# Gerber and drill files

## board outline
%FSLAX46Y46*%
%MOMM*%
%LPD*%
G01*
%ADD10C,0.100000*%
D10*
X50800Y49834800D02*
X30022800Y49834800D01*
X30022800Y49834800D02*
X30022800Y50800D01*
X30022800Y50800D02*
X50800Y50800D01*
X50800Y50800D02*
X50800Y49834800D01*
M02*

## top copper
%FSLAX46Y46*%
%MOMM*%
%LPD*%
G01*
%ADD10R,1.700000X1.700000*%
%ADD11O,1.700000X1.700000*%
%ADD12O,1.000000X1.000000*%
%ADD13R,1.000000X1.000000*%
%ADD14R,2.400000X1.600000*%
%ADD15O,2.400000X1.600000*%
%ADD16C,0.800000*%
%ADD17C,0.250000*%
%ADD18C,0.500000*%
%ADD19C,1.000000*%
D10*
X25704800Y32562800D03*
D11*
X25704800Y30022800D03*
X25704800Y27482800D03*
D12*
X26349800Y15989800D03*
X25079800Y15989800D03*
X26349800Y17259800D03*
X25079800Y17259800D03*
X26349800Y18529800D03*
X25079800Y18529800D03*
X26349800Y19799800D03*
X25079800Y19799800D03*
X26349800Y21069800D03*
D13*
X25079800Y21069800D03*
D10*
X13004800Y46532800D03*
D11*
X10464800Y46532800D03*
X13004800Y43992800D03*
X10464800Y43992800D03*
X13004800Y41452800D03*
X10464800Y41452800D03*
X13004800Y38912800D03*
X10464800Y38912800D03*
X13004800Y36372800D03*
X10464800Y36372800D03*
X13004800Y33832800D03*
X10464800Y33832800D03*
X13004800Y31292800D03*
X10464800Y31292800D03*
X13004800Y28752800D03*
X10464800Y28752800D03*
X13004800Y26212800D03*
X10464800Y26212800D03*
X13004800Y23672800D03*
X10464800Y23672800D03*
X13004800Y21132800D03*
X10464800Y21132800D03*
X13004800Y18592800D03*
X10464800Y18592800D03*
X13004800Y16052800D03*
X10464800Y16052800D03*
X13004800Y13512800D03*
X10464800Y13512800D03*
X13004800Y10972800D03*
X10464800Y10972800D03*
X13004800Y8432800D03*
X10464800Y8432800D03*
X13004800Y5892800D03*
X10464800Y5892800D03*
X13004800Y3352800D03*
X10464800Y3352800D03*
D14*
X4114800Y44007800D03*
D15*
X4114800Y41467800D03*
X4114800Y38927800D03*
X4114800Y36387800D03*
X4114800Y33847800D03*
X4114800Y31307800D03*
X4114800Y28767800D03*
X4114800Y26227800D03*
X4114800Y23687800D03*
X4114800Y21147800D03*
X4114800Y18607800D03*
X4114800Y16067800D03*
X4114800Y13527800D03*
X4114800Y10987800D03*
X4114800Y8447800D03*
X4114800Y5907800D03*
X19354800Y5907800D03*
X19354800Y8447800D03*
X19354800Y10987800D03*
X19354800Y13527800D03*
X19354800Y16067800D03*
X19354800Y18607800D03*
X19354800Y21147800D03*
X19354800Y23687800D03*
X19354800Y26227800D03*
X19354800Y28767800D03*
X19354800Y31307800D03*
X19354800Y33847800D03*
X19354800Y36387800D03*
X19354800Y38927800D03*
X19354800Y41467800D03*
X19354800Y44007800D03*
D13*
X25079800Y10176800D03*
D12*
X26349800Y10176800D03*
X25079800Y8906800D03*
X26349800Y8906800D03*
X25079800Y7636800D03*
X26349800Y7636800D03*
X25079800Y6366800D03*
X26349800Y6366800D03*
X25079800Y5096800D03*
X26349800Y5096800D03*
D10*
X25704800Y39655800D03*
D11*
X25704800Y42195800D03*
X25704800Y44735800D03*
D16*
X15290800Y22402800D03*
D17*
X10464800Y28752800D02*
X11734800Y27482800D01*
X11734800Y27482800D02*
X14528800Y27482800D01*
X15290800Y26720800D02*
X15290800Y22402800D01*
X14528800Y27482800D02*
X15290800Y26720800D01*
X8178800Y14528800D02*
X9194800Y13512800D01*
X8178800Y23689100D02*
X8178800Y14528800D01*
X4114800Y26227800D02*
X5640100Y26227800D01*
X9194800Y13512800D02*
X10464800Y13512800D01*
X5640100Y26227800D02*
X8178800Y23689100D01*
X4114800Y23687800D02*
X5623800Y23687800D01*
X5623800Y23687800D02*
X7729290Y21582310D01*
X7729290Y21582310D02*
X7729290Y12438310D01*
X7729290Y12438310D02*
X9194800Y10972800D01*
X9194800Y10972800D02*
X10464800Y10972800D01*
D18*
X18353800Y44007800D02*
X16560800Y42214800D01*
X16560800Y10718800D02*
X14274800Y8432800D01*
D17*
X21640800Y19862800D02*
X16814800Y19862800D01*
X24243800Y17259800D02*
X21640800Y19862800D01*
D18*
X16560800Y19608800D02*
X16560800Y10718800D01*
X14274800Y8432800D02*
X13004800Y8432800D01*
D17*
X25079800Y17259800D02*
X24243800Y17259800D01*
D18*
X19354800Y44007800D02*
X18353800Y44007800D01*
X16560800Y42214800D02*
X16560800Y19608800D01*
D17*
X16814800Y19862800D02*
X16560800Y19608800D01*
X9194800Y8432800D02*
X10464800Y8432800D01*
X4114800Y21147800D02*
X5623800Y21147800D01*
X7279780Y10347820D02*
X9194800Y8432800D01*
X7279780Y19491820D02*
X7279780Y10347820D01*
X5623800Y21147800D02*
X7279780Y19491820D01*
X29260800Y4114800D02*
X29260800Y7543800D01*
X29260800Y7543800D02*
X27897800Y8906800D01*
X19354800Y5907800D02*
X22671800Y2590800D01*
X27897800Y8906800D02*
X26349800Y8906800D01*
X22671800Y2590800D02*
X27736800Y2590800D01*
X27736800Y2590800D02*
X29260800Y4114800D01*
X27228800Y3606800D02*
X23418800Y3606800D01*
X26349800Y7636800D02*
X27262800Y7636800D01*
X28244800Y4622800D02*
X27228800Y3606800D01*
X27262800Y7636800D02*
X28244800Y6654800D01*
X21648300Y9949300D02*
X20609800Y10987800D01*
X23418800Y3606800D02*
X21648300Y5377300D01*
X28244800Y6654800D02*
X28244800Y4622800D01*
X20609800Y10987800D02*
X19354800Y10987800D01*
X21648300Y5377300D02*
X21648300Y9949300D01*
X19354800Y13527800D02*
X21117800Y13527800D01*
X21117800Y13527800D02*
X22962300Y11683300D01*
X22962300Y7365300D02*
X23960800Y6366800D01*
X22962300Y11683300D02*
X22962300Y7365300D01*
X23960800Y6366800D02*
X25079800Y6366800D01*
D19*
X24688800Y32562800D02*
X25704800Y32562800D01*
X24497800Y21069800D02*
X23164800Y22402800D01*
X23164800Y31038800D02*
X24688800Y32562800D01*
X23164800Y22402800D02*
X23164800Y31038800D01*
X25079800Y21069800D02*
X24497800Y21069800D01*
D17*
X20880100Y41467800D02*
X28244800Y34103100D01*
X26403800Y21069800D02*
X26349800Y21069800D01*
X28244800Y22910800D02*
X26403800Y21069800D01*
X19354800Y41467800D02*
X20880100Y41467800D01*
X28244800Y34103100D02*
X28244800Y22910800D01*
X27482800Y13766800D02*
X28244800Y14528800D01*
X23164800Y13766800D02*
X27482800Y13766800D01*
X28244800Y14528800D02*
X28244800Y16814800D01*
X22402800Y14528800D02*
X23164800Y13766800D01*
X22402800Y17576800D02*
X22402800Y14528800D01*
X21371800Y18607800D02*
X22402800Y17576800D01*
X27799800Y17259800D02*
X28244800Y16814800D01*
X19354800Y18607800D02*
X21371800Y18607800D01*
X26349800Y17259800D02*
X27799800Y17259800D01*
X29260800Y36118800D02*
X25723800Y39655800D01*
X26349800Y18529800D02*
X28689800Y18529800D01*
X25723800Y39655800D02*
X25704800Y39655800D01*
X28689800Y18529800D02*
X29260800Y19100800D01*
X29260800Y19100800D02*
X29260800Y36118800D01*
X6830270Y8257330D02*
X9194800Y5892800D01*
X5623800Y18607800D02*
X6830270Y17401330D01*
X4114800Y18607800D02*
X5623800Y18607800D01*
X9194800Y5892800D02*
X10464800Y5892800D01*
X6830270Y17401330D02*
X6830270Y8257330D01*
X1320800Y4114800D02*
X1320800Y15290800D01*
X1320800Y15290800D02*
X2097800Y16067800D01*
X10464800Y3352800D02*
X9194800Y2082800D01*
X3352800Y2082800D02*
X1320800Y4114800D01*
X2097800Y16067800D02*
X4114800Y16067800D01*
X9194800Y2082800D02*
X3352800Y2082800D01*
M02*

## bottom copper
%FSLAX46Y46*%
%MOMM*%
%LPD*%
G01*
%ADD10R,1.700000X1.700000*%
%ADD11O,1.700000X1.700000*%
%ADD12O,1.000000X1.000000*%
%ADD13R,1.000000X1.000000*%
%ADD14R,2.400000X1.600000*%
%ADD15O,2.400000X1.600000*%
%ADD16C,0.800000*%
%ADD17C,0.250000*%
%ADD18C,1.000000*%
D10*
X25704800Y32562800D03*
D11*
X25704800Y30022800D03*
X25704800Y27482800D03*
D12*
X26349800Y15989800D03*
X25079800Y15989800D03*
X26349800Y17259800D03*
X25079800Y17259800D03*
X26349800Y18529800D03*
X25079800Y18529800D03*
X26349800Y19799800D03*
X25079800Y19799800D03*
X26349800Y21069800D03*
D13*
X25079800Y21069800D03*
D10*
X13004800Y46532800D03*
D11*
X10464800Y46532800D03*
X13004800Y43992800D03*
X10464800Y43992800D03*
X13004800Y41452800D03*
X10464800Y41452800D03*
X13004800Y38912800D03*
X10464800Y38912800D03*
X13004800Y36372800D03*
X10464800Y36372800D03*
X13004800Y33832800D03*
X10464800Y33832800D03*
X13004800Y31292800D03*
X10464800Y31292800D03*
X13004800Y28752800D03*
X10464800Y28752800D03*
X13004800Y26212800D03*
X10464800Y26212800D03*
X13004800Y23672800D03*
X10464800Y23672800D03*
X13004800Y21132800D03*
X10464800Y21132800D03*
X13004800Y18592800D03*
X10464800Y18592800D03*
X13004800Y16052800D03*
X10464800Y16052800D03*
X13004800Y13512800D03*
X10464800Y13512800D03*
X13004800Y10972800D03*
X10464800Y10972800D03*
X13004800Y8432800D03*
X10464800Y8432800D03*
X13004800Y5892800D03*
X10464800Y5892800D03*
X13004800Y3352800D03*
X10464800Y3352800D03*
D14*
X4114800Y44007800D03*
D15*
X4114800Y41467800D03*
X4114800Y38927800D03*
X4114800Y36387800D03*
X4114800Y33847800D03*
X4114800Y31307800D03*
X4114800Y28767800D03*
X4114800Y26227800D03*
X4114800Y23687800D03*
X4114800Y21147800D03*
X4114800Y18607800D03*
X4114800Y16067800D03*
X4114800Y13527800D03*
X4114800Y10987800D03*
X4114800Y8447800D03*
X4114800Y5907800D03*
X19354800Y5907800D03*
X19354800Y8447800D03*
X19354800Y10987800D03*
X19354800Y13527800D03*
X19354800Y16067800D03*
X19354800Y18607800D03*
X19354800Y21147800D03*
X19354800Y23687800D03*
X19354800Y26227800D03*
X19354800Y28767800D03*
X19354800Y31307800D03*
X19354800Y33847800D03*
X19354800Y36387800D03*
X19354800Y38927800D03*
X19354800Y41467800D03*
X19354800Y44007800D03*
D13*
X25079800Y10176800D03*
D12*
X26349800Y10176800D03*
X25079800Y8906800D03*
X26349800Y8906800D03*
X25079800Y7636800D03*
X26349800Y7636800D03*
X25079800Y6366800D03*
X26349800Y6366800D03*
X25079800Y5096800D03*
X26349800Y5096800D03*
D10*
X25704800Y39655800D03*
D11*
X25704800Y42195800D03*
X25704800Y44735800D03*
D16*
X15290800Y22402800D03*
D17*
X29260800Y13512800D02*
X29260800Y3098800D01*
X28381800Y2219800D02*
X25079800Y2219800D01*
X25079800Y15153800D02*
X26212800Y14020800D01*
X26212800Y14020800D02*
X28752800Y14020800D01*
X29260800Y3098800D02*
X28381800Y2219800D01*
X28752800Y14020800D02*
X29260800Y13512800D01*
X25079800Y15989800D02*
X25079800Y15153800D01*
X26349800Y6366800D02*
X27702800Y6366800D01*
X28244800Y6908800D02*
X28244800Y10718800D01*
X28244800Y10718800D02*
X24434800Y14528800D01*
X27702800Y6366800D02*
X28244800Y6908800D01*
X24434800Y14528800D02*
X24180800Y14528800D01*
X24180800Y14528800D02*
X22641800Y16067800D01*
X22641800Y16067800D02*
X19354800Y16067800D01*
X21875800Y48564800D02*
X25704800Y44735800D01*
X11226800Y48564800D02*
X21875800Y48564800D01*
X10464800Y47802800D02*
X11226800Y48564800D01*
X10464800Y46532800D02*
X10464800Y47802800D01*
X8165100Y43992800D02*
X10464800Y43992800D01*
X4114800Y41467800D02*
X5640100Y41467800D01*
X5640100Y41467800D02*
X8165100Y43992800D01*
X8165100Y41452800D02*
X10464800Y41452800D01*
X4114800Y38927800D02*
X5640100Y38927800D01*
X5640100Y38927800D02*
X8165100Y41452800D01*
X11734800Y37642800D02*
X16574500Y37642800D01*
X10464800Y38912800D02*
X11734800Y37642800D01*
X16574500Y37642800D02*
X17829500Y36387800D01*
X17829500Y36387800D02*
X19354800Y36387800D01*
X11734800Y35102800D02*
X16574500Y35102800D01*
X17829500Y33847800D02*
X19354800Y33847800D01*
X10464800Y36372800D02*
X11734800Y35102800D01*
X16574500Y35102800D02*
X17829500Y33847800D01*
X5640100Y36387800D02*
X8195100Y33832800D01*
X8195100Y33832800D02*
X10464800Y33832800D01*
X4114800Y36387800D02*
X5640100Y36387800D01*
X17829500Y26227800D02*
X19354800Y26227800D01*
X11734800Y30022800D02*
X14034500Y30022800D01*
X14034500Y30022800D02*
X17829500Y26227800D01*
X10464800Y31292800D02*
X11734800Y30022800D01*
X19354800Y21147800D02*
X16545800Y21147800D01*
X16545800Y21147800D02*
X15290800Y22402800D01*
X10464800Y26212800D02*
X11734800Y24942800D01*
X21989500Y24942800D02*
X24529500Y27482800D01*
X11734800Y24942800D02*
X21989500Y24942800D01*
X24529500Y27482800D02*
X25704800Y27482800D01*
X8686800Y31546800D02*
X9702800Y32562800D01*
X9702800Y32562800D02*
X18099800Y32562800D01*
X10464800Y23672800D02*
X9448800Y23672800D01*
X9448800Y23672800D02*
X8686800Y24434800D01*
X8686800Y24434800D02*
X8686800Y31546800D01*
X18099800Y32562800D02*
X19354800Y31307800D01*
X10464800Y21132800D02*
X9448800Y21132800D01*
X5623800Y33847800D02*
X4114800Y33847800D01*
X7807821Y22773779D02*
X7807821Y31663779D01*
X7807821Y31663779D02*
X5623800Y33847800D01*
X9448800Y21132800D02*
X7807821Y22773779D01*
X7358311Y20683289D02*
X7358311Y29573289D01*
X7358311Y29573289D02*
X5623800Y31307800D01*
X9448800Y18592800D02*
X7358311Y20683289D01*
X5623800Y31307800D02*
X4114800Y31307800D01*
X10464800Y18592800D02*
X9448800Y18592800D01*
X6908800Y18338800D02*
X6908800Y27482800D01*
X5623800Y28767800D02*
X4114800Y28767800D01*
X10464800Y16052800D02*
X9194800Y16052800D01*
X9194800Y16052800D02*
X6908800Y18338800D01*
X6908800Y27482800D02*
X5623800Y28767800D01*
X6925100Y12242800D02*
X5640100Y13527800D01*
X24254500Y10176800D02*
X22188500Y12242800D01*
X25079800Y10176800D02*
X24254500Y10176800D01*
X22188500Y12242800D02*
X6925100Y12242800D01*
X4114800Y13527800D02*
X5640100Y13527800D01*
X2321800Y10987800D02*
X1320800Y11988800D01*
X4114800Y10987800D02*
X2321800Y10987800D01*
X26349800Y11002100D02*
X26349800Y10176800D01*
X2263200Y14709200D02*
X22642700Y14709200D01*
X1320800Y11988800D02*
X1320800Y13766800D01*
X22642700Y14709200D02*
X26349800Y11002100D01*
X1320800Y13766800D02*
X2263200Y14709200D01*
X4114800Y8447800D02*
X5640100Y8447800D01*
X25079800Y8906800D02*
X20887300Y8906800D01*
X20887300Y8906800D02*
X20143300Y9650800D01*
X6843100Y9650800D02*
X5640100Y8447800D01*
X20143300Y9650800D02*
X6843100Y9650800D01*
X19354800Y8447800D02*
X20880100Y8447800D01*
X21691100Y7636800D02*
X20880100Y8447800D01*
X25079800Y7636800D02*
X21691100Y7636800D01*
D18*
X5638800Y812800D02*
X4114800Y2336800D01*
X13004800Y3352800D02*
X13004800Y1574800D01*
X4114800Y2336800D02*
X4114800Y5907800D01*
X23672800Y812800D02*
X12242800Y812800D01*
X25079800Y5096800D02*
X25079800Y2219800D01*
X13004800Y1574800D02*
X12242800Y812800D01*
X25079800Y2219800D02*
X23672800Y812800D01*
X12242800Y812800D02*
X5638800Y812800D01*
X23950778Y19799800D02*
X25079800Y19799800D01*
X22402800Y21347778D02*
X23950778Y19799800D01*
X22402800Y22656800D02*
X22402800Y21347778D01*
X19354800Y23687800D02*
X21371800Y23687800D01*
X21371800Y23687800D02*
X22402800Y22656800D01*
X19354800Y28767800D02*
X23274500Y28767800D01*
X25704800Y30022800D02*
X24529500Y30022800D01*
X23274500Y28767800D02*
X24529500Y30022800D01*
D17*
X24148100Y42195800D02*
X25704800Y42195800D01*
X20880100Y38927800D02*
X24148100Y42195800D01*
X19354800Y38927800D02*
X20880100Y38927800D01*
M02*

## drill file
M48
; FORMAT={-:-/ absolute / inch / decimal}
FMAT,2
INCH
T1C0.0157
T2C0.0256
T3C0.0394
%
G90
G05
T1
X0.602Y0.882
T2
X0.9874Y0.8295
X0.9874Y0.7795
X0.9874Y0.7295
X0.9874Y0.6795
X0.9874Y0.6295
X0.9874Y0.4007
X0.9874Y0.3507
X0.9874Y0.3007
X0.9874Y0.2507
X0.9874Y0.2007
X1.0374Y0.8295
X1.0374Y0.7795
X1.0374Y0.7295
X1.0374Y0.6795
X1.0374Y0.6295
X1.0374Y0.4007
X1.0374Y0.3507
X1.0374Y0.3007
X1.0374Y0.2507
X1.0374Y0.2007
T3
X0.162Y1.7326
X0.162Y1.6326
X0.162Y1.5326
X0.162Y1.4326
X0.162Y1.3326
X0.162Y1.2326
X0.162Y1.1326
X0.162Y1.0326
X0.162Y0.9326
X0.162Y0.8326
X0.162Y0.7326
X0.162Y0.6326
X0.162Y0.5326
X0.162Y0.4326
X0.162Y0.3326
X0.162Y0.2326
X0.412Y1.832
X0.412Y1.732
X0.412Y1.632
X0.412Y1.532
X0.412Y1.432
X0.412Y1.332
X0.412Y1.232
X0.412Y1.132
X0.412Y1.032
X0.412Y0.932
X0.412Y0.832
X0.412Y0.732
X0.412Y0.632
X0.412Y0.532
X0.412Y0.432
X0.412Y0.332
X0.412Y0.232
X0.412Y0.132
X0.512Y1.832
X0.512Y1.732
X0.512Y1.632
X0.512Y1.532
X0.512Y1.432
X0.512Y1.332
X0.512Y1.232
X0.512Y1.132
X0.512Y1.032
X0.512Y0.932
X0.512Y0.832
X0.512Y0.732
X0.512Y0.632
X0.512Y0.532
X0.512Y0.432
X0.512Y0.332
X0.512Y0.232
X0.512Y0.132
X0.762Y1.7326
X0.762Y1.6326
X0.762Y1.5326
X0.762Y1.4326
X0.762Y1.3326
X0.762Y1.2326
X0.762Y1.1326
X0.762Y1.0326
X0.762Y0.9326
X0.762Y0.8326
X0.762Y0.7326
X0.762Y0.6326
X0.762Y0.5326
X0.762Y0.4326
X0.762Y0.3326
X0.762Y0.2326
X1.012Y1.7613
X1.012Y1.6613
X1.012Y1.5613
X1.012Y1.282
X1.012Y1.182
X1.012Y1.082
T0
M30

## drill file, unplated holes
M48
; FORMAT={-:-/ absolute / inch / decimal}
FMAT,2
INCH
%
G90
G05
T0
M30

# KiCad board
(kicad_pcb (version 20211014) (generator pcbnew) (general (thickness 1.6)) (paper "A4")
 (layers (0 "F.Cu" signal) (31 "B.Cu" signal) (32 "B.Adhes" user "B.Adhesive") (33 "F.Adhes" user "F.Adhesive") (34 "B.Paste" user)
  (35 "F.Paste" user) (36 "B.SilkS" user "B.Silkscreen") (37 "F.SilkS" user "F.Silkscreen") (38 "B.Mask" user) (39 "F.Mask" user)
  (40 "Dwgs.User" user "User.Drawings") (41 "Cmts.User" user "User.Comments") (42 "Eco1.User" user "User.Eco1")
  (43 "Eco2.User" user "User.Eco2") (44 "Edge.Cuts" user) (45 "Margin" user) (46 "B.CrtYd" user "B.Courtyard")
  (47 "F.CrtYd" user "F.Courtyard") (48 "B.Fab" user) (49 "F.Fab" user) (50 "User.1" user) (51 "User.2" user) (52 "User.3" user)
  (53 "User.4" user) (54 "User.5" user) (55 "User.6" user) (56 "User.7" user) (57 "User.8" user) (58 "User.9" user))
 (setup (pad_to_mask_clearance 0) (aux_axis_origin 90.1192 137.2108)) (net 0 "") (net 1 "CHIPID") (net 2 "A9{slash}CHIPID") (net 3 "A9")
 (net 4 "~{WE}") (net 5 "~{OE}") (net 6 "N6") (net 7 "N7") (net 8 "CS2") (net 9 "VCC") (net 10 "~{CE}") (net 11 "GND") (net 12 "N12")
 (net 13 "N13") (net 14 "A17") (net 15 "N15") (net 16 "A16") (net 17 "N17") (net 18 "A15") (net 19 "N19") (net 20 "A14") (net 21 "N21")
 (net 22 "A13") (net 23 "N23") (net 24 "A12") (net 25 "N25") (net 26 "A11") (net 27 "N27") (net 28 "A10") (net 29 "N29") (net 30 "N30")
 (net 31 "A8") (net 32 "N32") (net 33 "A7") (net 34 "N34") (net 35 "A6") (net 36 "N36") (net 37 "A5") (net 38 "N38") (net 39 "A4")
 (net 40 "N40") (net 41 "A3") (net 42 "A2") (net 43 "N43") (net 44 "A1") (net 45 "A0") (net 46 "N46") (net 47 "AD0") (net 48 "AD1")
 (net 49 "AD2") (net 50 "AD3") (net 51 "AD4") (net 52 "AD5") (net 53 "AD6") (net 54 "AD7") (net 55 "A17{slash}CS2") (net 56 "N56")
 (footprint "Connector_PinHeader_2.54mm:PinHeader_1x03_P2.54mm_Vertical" (layer "F.Cu") (at 115.824 104.648)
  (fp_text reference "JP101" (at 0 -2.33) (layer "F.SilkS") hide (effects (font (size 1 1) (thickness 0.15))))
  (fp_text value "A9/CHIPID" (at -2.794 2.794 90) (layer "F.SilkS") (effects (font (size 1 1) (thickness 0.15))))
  (pad "1" thru_hole rect (at 0 0) (size 1.7 1.7) (drill 1) (layers *.Cu *.Mask) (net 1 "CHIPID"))
  (pad "2" thru_hole oval (at 0 2.54) (size 1.7 1.7) (drill 1) (layers *.Cu *.Mask) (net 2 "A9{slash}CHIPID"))
  (pad "3" thru_hole oval (at 0 5.08) (size 1.7 1.7) (drill 1) (layers *.Cu *.Mask) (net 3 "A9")))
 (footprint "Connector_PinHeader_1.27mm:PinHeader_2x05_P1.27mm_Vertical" (layer "F.Cu") (at 115.199 116.141)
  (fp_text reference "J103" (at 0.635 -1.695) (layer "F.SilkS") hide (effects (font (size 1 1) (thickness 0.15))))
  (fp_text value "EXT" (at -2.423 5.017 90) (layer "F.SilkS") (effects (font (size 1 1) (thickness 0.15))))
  (pad "1" thru_hole rect (at 0 0) (size 1 1) (drill 0.65) (layers *.Cu *.Mask) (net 1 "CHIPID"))
  (pad "2" thru_hole oval (at 1.27 0) (size 1 1) (drill 0.65) (layers *.Cu *.Mask) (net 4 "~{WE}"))
  (pad "3" thru_hole oval (at 0 1.27) (size 1 1) (drill 0.65) (layers *.Cu *.Mask) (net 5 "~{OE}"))
  (pad "4" thru_hole oval (at 1.27 1.27) (size 1 1) (drill 0.65) (layers *.Cu *.Mask) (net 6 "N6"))
  (pad "5" thru_hole oval (at 0 2.54) (size 1 1) (drill 0.65) (layers *.Cu *.Mask) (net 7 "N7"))
  (pad "6" thru_hole oval (at 1.27 2.54) (size 1 1) (drill 0.65) (layers *.Cu *.Mask) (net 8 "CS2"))
  (pad "7" thru_hole oval (at 0 3.81) (size 1 1) (drill 0.65) (layers *.Cu *.Mask) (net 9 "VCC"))
  (pad "8" thru_hole oval (at 1.27 3.81) (size 1 1) (drill 0.65) (layers *.Cu *.Mask) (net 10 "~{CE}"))
  (pad "9" thru_hole oval (at 0 5.08) (size 1 1) (drill 0.65) (layers *.Cu *.Mask) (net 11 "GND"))
  (pad "10" thru_hole oval (at 1.27 5.08) (size 1 1) (drill 0.65) (layers *.Cu *.Mask) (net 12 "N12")))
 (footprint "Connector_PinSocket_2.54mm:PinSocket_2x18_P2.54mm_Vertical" (layer "F.Cu") (at 103.124 90.678)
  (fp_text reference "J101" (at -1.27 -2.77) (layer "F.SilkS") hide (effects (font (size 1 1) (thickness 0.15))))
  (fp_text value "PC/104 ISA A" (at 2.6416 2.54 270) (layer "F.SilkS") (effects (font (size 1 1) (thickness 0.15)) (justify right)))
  (pad "1" thru_hole rect (at 0 0) (size 1.7 1.7) (drill 1) (layers *.Cu *.Mask) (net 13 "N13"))
  (pad "2" thru_hole oval (at -2.54 0) (size 1.7 1.7) (drill 1) (layers *.Cu *.Mask) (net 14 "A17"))
  (pad "3" thru_hole oval (at 0 2.54) (size 1.7 1.7) (drill 1) (layers *.Cu *.Mask) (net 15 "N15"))
  (pad "4" thru_hole oval (at -2.54 2.54) (size 1.7 1.7) (drill 1) (layers *.Cu *.Mask) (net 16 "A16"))
  (pad "5" thru_hole oval (at 0 5.08) (size 1.7 1.7) (drill 1) (layers *.Cu *.Mask) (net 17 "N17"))
  (pad "6" thru_hole oval (at -2.54 5.08) (size 1.7 1.7) (drill 1) (layers *.Cu *.Mask) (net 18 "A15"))
  (pad "7" thru_hole oval (at 0 7.62) (size 1.7 1.7) (drill 1) (layers *.Cu *.Mask) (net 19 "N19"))
  (pad "8" thru_hole oval (at -2.54 7.62) (size 1.7 1.7) (drill 1) (layers *.Cu *.Mask) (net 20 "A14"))
  (pad "9" thru_hole oval (at 0 10.16) (size 1.7 1.7) (drill 1) (layers *.Cu *.Mask) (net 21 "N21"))
  (pad "10" thru_hole oval (at -2.54 10.16) (size 1.7 1.7) (drill 1) (layers *.Cu *.Mask) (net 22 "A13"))
  (pad "11" thru_hole oval (at 0 12.7) (size 1.7 1.7) (drill 1) (layers *.Cu *.Mask) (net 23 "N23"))
  (pad "12" thru_hole oval (at -2.54 12.7) (size 1.7 1.7) (drill 1) (layers *.Cu *.Mask) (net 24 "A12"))
  (pad "13" thru_hole oval (at 0 15.24) (size 1.7 1.7) (drill 1) (layers *.Cu *.Mask) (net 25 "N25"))
  (pad "14" thru_hole oval (at -2.54 15.24) (size 1.7 1.7) (drill 1) (layers *.Cu *.Mask) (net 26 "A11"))
  (pad "15" thru_hole oval (at 0 17.78) (size 1.7 1.7) (drill 1) (layers *.Cu *.Mask) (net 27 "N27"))
  (pad "16" thru_hole oval (at -2.54 17.78) (size 1.7 1.7) (drill 1) (layers *.Cu *.Mask) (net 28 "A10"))
  (pad "17" thru_hole oval (at 0 20.32) (size 1.7 1.7) (drill 1) (layers *.Cu *.Mask) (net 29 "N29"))
  (pad "18" thru_hole oval (at -2.54 20.32) (size 1.7 1.7) (drill 1) (layers *.Cu *.Mask) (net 3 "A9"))
  (pad "19" thru_hole oval (at 0 22.86) (size 1.7 1.7) (drill 1) (layers *.Cu *.Mask) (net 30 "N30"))
  (pad "20" thru_hole oval (at -2.54 22.86) (size 1.7 1.7) (drill 1) (layers *.Cu *.Mask) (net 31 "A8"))
  (pad "21" thru_hole oval (at 0 25.4) (size 1.7 1.7) (drill 1) (layers *.Cu *.Mask) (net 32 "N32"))
  (pad "22" thru_hole oval (at -2.54 25.4) (size 1.7 1.7) (drill 1) (layers *.Cu *.Mask) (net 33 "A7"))
  (pad "23" thru_hole oval (at 0 27.94) (size 1.7 1.7) (drill 1) (layers *.Cu *.Mask) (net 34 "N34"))
  (pad "24" thru_hole oval (at -2.54 27.94) (size 1.7 1.7) (drill 1) (layers *.Cu *.Mask) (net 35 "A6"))
  (pad "25" thru_hole oval (at 0 30.48) (size 1.7 1.7) (drill 1) (layers *.Cu *.Mask) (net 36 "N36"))
  (pad "26" thru_hole oval (at -2.54 30.48) (size 1.7 1.7) (drill 1) (layers *.Cu *.Mask) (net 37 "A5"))
  (pad "27" thru_hole oval (at 0 33.02) (size 1.7 1.7) (drill 1) (layers *.Cu *.Mask) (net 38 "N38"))
  (pad "28" thru_hole oval (at -2.54 33.02) (size 1.7 1.7) (drill 1) (layers *.Cu *.Mask) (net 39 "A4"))
  (pad "29" thru_hole oval (at 0 35.56) (size 1.7 1.7) (drill 1) (layers *.Cu *.Mask) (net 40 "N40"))
  (pad "30" thru_hole oval (at -2.54 35.56) (size 1.7 1.7) (drill 1) (layers *.Cu *.Mask) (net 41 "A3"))
  (pad "31" thru_hole oval (at 0 38.1) (size 1.7 1.7) (drill 1) (layers *.Cu *.Mask) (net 9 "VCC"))
  (pad "32" thru_hole oval (at -2.54 38.1) (size 1.7 1.7) (drill 1) (layers *.Cu *.Mask) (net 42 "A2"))
  (pad "33" thru_hole oval (at 0 40.64) (size 1.7 1.7) (drill 1) (layers *.Cu *.Mask) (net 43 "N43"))
  (pad "34" thru_hole oval (at -2.54 40.64) (size 1.7 1.7) (drill 1) (layers *.Cu *.Mask) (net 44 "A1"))
  (pad "35" thru_hole oval (at 0 43.18) (size 1.7 1.7) (drill 1) (layers *.Cu *.Mask) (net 11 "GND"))
  (pad "36" thru_hole oval (at -2.54 43.18) (size 1.7 1.7) (drill 1) (layers *.Cu *.Mask) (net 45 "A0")))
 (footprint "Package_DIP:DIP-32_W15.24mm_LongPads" (layer "F.Cu") (at 94.234 93.203)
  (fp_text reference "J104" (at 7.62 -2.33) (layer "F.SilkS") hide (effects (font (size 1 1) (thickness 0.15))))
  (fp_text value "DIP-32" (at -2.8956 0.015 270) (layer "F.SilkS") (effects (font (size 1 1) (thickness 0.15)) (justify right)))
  (pad "1" thru_hole rect (at 0 0) (size 2.4 1.6) (drill 1) (layers *.Cu *.Mask) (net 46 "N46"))
  (pad "2" thru_hole oval (at 0 2.54) (size 2.4 1.6) (drill 1) (layers *.Cu *.Mask) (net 16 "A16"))
  (pad "3" thru_hole oval (at 0 5.08) (size 2.4 1.6) (drill 1) (layers *.Cu *.Mask) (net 18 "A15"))
  (pad "4" thru_hole oval (at 0 7.62) (size 2.4 1.6) (drill 1) (layers *.Cu *.Mask) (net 24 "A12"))
  (pad "5" thru_hole oval (at 0 10.16) (size 2.4 1.6) (drill 1) (layers *.Cu *.Mask) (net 33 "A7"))
  (pad "6" thru_hole oval (at 0 12.7) (size 2.4 1.6) (drill 1) (layers *.Cu *.Mask) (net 35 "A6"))
  (pad "7" thru_hole oval (at 0 15.24) (size 2.4 1.6) (drill 1) (layers *.Cu *.Mask) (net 37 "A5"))
  (pad "8" thru_hole oval (at 0 17.78) (size 2.4 1.6) (drill 1) (layers *.Cu *.Mask) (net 39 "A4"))
  (pad "9" thru_hole oval (at 0 20.32) (size 2.4 1.6) (drill 1) (layers *.Cu *.Mask) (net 41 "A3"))
  (pad "10" thru_hole oval (at 0 22.86) (size 2.4 1.6) (drill 1) (layers *.Cu *.Mask) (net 42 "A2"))
  (pad "11" thru_hole oval (at 0 25.4) (size 2.4 1.6) (drill 1) (layers *.Cu *.Mask) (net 44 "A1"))
  (pad "12" thru_hole oval (at 0 27.94) (size 2.4 1.6) (drill 1) (layers *.Cu *.Mask) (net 45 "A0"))
  (pad "13" thru_hole oval (at 0 30.48) (size 2.4 1.6) (drill 1) (layers *.Cu *.Mask) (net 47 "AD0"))
  (pad "14" thru_hole oval (at 0 33.02) (size 2.4 1.6) (drill 1) (layers *.Cu *.Mask) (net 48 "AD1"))
  (pad "15" thru_hole oval (at 0 35.56) (size 2.4 1.6) (drill 1) (layers *.Cu *.Mask) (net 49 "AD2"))
  (pad "16" thru_hole oval (at 0 38.1) (size 2.4 1.6) (drill 1) (layers *.Cu *.Mask) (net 11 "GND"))
  (pad "17" thru_hole oval (at 15.24 38.1) (size 2.4 1.6) (drill 1) (layers *.Cu *.Mask) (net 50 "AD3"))
  (pad "18" thru_hole oval (at 15.24 35.56) (size 2.4 1.6) (drill 1) (layers *.Cu *.Mask) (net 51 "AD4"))
  (pad "19" thru_hole oval (at 15.24 33.02) (size 2.4 1.6) (drill 1) (layers *.Cu *.Mask) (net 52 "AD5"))
  (pad "20" thru_hole oval (at 15.24 30.48) (size 2.4 1.6) (drill 1) (layers *.Cu *.Mask) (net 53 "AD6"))
  (pad "21" thru_hole oval (at 15.24 27.94) (size 2.4 1.6) (drill 1) (layers *.Cu *.Mask) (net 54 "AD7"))
  (pad "22" thru_hole oval (at 15.24 25.4) (size 2.4 1.6) (drill 1) (layers *.Cu *.Mask) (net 10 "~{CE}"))
  (pad "23" thru_hole oval (at 15.24 22.86) (size 2.4 1.6) (drill 1) (layers *.Cu *.Mask) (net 28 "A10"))
  (pad "24" thru_hole oval (at 15.24 20.32) (size 2.4 1.6) (drill 1) (layers *.Cu *.Mask) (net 5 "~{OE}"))
  (pad "25" thru_hole oval (at 15.24 17.78) (size 2.4 1.6) (drill 1) (layers *.Cu *.Mask) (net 26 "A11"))
  (pad "26" thru_hole oval (at 15.24 15.24) (size 2.4 1.6) (drill 1) (layers *.Cu *.Mask) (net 2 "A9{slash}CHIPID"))
  (pad "27" thru_hole oval (at 15.24 12.7) (size 2.4 1.6) (drill 1) (layers *.Cu *.Mask) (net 31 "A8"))
  (pad "28" thru_hole oval (at 15.24 10.16) (size 2.4 1.6) (drill 1) (layers *.Cu *.Mask) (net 22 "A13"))
  (pad "29" thru_hole oval (at 15.24 7.62) (size 2.4 1.6) (drill 1) (layers *.Cu *.Mask) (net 20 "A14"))
  (pad "30" thru_hole oval (at 15.24 5.08) (size 2.4 1.6) (drill 1) (layers *.Cu *.Mask) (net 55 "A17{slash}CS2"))
  (pad "31" thru_hole oval (at 15.24 2.54) (size 2.4 1.6) (drill 1) (layers *.Cu *.Mask) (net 4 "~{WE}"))
  (pad "32" thru_hole oval (at 15.24 0) (size 2.4 1.6) (drill 1) (layers *.Cu *.Mask) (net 9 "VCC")))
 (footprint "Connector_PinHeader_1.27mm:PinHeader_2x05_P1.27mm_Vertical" (layer "F.Cu") (at 115.199 127.034)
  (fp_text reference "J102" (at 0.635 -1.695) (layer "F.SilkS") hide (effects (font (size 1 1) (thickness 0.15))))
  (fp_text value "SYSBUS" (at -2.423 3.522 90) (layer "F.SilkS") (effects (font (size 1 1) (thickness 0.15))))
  (pad "1" thru_hole rect (at 0 0) (size 1 1) (drill 0.65) (layers *.Cu *.Mask) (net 47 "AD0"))
  (pad "2" thru_hole oval (at 1.27 0) (size 1 1) (drill 0.65) (layers *.Cu *.Mask) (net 48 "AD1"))
  (pad "3" thru_hole oval (at 0 1.27) (size 1 1) (drill 0.65) (layers *.Cu *.Mask) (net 49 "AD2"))
  (pad "4" thru_hole oval (at 1.27 1.27) (size 1 1) (drill 0.65) (layers *.Cu *.Mask) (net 50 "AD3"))
  (pad "5" thru_hole oval (at 0 2.54) (size 1 1) (drill 0.65) (layers *.Cu *.Mask) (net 51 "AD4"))
  (pad "6" thru_hole oval (at 1.27 2.54) (size 1 1) (drill 0.65) (layers *.Cu *.Mask) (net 52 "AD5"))
  (pad "7" thru_hole oval (at 0 3.81) (size 1 1) (drill 0.65) (layers *.Cu *.Mask) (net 53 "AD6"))
  (pad "8" thru_hole oval (at 1.27 3.81) (size 1 1) (drill 0.65) (layers *.Cu *.Mask) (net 54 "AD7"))
  (pad "9" thru_hole oval (at 0 5.08) (size 1 1) (drill 0.65) (layers *.Cu *.Mask) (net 11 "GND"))
  (pad "10" thru_hole oval (at 1.27 5.08) (size 1 1) (drill 0.65) (layers *.Cu *.Mask) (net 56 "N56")))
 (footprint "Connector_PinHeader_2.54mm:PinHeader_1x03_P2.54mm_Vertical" (layer "F.Cu") (at 115.824 97.555 180)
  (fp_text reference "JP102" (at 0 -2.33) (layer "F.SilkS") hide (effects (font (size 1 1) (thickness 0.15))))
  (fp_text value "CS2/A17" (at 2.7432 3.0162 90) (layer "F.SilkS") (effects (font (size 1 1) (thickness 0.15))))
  (pad "1" thru_hole rect (at 0 0 180) (size 1.7 1.7) (drill 1) (layers *.Cu *.Mask) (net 8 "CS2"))
  (pad "2" thru_hole oval (at 0 2.54 180) (size 1.7 1.7) (drill 1) (layers *.Cu *.Mask) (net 55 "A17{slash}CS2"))
  (pad "3" thru_hole oval (at 0 5.08 180) (size 1.7 1.7) (drill 1) (layers *.Cu *.Mask) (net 14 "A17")))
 (gr_line (start 120.142 137.16) (end 90.17 137.16) (layer "Edge.Cuts") (width 0.1))
 (gr_arc (start 92.760799 89.916) (mid 92.020197 91.781074) (end 90.17 92.558097) (layer "Edge.Cuts") (width 0.1))
 (gr_line (start 92.7608 87.376) (end 92.760799 89.916) (layer "Edge.Cuts") (width 0.1))
 (gr_line (start 120.142 87.376) (end 120.142 137.16) (layer "Edge.Cuts") (width 0.1))
 (gr_line (start 90.17 137.16) (end 90.17 92.558097) (layer "Edge.Cuts") (width 0.1))
 (gr_line (start 92.7608 87.376) (end 120.142 87.376) (layer "Edge.Cuts") (width 0.1))
 (segment (start 111.995 88.646) (end 115.824 92.475) (width 0.25) (layer "B.Cu") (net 14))
 (segment (start 101.346 88.646) (end 111.995 88.646) (width 0.25) (layer "B.Cu") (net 14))
 (segment (start 100.584 89.408) (end 101.346 88.646) (width 0.25) (layer "B.Cu") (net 14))
 (segment (start 100.584 90.678) (end 100.584 89.408) (width 0.25) (layer "B.Cu") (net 14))
 (segment (start 98.2843 93.218) (end 100.584 93.218) (width 0.25) (layer "B.Cu") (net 16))
 (segment (start 94.234 95.743) (end 95.7593 95.743) (width 0.25) (layer "B.Cu") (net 16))
 (segment (start 95.7593 95.743) (end 98.2843 93.218) (width 0.25) (layer "B.Cu") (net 16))
 (segment (start 98.2843 95.758) (end 100.584 95.758) (width 0.25) (layer "B.Cu") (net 18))
 (segment (start 94.234 98.283) (end 95.7593 98.283) (width 0.25) (layer "B.Cu") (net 18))
 (segment (start 95.7593 98.283) (end 98.2843 95.758) (width 0.25) (layer "B.Cu") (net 18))
 (segment (start 101.854 99.568) (end 106.6937 99.568) (width 0.25) (layer "B.Cu") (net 20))
 (segment (start 100.584 98.298) (end 101.854 99.568) (width 0.25) (layer "B.Cu") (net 20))
 (segment (start 106.6937 99.568) (end 107.9487 100.823) (width 0.25) (layer "B.Cu") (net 20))
 (segment (start 107.9487 100.823) (end 109.474 100.823) (width 0.25) (layer "B.Cu") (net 20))
 (segment (start 101.854 102.108) (end 106.6937 102.108) (width 0.25) (layer "B.Cu") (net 22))
 (segment (start 107.9487 103.363) (end 109.474 103.363) (width 0.25) (layer "B.Cu") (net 22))
 (segment (start 100.584 100.838) (end 101.854 102.108) (width 0.25) (layer "B.Cu") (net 22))
 (segment (start 106.6937 102.108) (end 107.9487 103.363) (width 0.25) (layer "B.Cu") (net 22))
 (segment (start 95.7593 100.823) (end 98.3143 103.378) (width 0.25) (layer "B.Cu") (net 24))
 (segment (start 98.3143 103.378) (end 100.584 103.378) (width 0.25) (layer "B.Cu") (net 24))
 (segment (start 94.234 100.823) (end 95.7593 100.823) (width 0.25) (layer "B.Cu") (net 24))
 (segment (start 107.9487 110.983) (end 109.474 110.983) (width 0.25) (layer "B.Cu") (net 26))
 (segment (start 101.854 107.188) (end 104.1537 107.188) (width 0.25) (layer "B.Cu") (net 26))
 (segment (start 104.1537 107.188) (end 107.9487 110.983) (width 0.25) (layer "B.Cu") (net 26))
 (segment (start 100.584 105.918) (end 101.854 107.188) (width 0.25) (layer "B.Cu") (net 26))
 (segment (start 100.584 108.458) (end 101.854 109.728) (width 0.25) (layer "F.Cu") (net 28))
 (segment (start 101.854 109.728) (end 104.648 109.728) (width 0.25) (layer "F.Cu") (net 28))
 (segment (start 105.41 110.49) (end 105.41 114.808) (width 0.25) (layer "F.Cu") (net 28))
 (segment (start 104.648 109.728) (end 105.41 110.49) (width 0.25) (layer "F.Cu") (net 28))
 (via (at 105.41 114.808) (size 0.8) (drill 0.4) (layers "F.Cu" "B.Cu") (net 28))
 (segment (start 109.474 116.063) (end 106.665 116.063) (width 0.25) (layer "B.Cu") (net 28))
 (segment (start 106.665 116.063) (end 105.41 114.808) (width 0.25) (layer "B.Cu") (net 28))
 (segment (start 100.584 110.998) (end 101.854 112.268) (width 0.25) (layer "B.Cu") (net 3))
 (segment (start 112.1087 112.268) (end 114.6487 109.728) (width 0.25) (layer "B.Cu") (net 3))
 (segment (start 101.854 112.268) (end 112.1087 112.268) (width 0.25) (layer "B.Cu") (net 3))
 (segment (start 114.6487 109.728) (end 115.824 109.728) (width 0.25) (layer "B.Cu") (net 3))
 (segment (start 98.806 105.664) (end 99.822 104.648) (width 0.25) (layer "B.Cu") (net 31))
 (segment (start 99.822 104.648) (end 108.219 104.648) (width 0.25) (layer "B.Cu") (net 31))
 (segment (start 100.584 113.538) (end 99.568 113.538) (width 0.25) (layer "B.Cu") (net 31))
 (segment (start 99.568 113.538) (end 98.806 112.776) (width 0.25) (layer "B.Cu") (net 31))
 (segment (start 98.806 112.776) (end 98.806 105.664) (width 0.25) (layer "B.Cu") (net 31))
 (segment (start 108.219 104.648) (end 109.474 105.903) (width 0.25) (layer "B.Cu") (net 31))
 (segment (start 100.584 116.078) (end 99.568 116.078) (width 0.25) (layer "B.Cu") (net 33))
 (segment (start 95.743 103.363) (end 94.234 103.363) (width 0.25) (layer "B.Cu") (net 33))
 (segment (start 97.927021 114.437021) (end 97.927021 105.547021) (width 0.25) (layer "B.Cu") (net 33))
 (segment (start 97.927021 105.547021) (end 95.743 103.363) (width 0.25) (layer "B.Cu") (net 33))
 (segment (start 99.568 116.078) (end 97.927021 114.437021) (width 0.25) (layer "B.Cu") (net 33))
 (segment (start 97.477511 116.527511) (end 97.477511 107.637511) (width 0.25) (layer "B.Cu") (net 35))
 (segment (start 97.477511 107.637511) (end 95.743 105.903) (width 0.25) (layer "B.Cu") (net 35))
 (segment (start 99.568 118.618) (end 97.477511 116.527511) (width 0.25) (layer "B.Cu") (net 35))
 (segment (start 95.743 105.903) (end 94.234 105.903) (width 0.25) (layer "B.Cu") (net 35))
 (segment (start 100.584 118.618) (end 99.568 118.618) (width 0.25) (layer "B.Cu") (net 35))
 (segment (start 97.028 118.872) (end 97.028 109.728) (width 0.25) (layer "B.Cu") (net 37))
 (segment (start 95.743 108.443) (end 94.234 108.443) (width 0.25) (layer "B.Cu") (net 37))
 (segment (start 100.584 121.158) (end 99.314 121.158) (width 0.25) (layer "B.Cu") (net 37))
 (segment (start 99.314 121.158) (end 97.028 118.872) (width 0.25) (layer "B.Cu") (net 37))
 (segment (start 97.028 109.728) (end 95.743 108.443) (width 0.25) (layer "B.Cu") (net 37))
 (segment (start 98.298 122.682) (end 99.314 123.698) (width 0.25) (layer "F.Cu") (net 39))
 (segment (start 98.298 113.5217) (end 98.298 122.682) (width 0.25) (layer "F.Cu") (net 39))
 (segment (start 94.234 110.983) (end 95.7593 110.983) (width 0.25) (layer "F.Cu") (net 39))
 (segment (start 99.314 123.698) (end 100.584 123.698) (width 0.25) (layer "F.Cu") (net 39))
 (segment (start 95.7593 110.983) (end 98.298 113.5217) (width 0.25) (layer "F.Cu") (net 39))
 (segment (start 94.234 113.523) (end 95.743 113.523) (width 0.25) (layer "F.Cu") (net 41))
 (segment (start 95.743 113.523) (end 97.84849 115.62849) (width 0.25) (layer "F.Cu") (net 41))
 (segment (start 97.84849 115.62849) (end 97.84849 124.77249) (width 0.25) (layer "F.Cu") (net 41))
 (segment (start 97.84849 124.77249) (end 99.314 126.238) (width 0.25) (layer "F.Cu") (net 41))
 (segment (start 99.314 126.238) (end 100.584 126.238) (width 0.25) (layer "F.Cu") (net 41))
 (segment (start 108.473 93.203) (end 106.68 94.996) (width 0.5) (layer "F.Cu") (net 9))
 (segment (start 106.68 126.492) (end 104.394 128.778) (width 0.5) (layer "F.Cu") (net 9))
 (segment (start 111.76 117.348) (end 106.934 117.348) (width 0.25) (layer "F.Cu") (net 9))
 (segment (start 114.363 119.951) (end 111.76 117.348) (width 0.25) (layer "F.Cu") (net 9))
 (segment (start 106.68 117.602) (end 106.68 126.492) (width 0.5) (layer "F.Cu") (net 9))
 (segment (start 104.394 128.778) (end 103.124 128.778) (width 0.5) (layer "F.Cu") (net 9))
 (segment (start 115.199 119.951) (end 114.363 119.951) (width 0.25) (layer "F.Cu") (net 9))
 (segment (start 109.474 93.203) (end 108.473 93.203) (width 0.5) (layer "F.Cu") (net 9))
 (segment (start 106.68 94.996) (end 106.68 117.602) (width 0.5) (layer "F.Cu") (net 9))
 (segment (start 106.934 117.348) (end 106.68 117.602) (width 0.25) (layer "F.Cu") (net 9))
 (segment (start 99.314 128.778) (end 100.584 128.778) (width 0.25) (layer "F.Cu") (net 42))
 (segment (start 94.234 116.063) (end 95.743 116.063) (width 0.25) (layer "F.Cu") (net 42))
 (segment (start 97.39898 126.86298) (end 99.314 128.778) (width 0.25) (layer "F.Cu") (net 42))
 (segment (start 97.39898 117.71898) (end 97.39898 126.86298) (width 0.25) (layer "F.Cu") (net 42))
 (segment (start 95.743 116.063) (end 97.39898 117.71898) (width 0.25) (layer "F.Cu") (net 42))
 (segment (start 97.0443 124.968) (end 95.7593 123.683) (width 0.25) (layer "B.Cu") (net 47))
 (segment (start 114.3737 127.034) (end 112.3077 124.968) (width 0.25) (layer "B.Cu") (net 47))
 (segment (start 115.199 127.034) (end 114.3737 127.034) (width 0.25) (layer "B.Cu") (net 47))
 (segment (start 112.3077 124.968) (end 97.0443 124.968) (width 0.25) (layer "B.Cu") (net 47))
 (segment (start 94.234 123.683) (end 95.7593 123.683) (width 0.25) (layer "B.Cu") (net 47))
 (segment (start 92.441 126.223) (end 91.44 125.222) (width 0.25) (layer "B.Cu") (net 48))
 (segment (start 94.234 126.223) (end 92.441 126.223) (width 0.25) (layer "B.Cu") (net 48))
 (segment (start 116.469 126.2087) (end 116.469 127.034) (width 0.25) (layer "B.Cu") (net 48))
 (segment (start 92.3824 122.5016) (end 112.7619 122.5016) (width 0.25) (layer "B.Cu") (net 48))
 (segment (start 91.44 125.222) (end 91.44 123.444) (width 0.25) (layer "B.Cu") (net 48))
 (segment (start 112.7619 122.5016) (end 116.469 126.2087) (width 0.25) (layer "B.Cu") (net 48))
 (segment (start 91.44 123.444) (end 92.3824 122.5016) (width 0.25) (layer "B.Cu") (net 48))
 (segment (start 94.234 128.763) (end 95.7593 128.763) (width 0.25) (layer "B.Cu") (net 49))
 (segment (start 115.199 128.304) (end 111.0065 128.304) (width 0.25) (layer "B.Cu") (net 49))
 (segment (start 111.0065 128.304) (end 110.2625 127.56) (width 0.25) (layer "B.Cu") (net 49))
 (segment (start 96.9623 127.56) (end 95.7593 128.763) (width 0.25) (layer "B.Cu") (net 49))
 (segment (start 110.2625 127.56) (end 96.9623 127.56) (width 0.25) (layer "B.Cu") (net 49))
 (segment (start 119.38 133.096) (end 119.38 129.667) (width 0.25) (layer "F.Cu") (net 50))
 (segment (start 119.38 129.667) (end 118.017 128.304) (width 0.25) (layer "F.Cu") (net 50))
 (segment (start 109.474 131.303) (end 112.791 134.62) (width 0.25) (layer "F.Cu") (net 50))
 (segment (start 118.017 128.304) (end 116.469 128.304) (width 0.25) (layer "F.Cu") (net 50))
 (segment (start 112.791 134.62) (end 117.856 134.62) (width 0.25) (layer "F.Cu") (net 50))
 (segment (start 117.856 134.62) (end 119.38 133.096) (width 0.25) (layer "F.Cu") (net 50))
 (segment (start 109.474 128.763) (end 110.9993 128.763) (width 0.25) (layer "B.Cu") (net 51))
 (segment (start 111.8103 129.574) (end 110.9993 128.763) (width 0.25) (layer "B.Cu") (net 51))
 (segment (start 115.199 129.574) (end 111.8103 129.574) (width 0.25) (layer "B.Cu") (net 51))
 (segment (start 117.348 133.604) (end 113.538 133.604) (width 0.25) (layer "F.Cu") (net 52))
 (segment (start 116.469 129.574) (end 117.382 129.574) (width 0.25) (layer "F.Cu") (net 52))
 (segment (start 118.364 132.588) (end 117.348 133.604) (width 0.25) (layer "F.Cu") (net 52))
 (segment (start 117.382 129.574) (end 118.364 130.556) (width 0.25) (layer "F.Cu") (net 52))
 (segment (start 111.7675 127.2615) (end 110.729 126.223) (width 0.25) (layer "F.Cu") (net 52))
 (segment (start 113.538 133.604) (end 111.7675 131.8335) (width 0.25) (layer "F.Cu") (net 52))
 (segment (start 118.364 130.556) (end 118.364 132.588) (width 0.25) (layer "F.Cu") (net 52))
 (segment (start 110.729 126.223) (end 109.474 126.223) (width 0.25) (layer "F.Cu") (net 52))
 (segment (start 111.7675 131.8335) (end 111.7675 127.2615) (width 0.25) (layer "F.Cu") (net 52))
 (segment (start 109.474 123.683) (end 111.237 123.683) (width 0.25) (layer "F.Cu") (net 53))
 (segment (start 111.237 123.683) (end 113.0815 125.5275) (width 0.25) (layer "F.Cu") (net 53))
 (segment (start 113.0815 129.8455) (end 114.08 130.844) (width 0.25) (layer "F.Cu") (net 53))
 (segment (start 113.0815 125.5275) (end 113.0815 129.8455) (width 0.25) (layer "F.Cu") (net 53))
 (segment (start 114.08 130.844) (end 115.199 130.844) (width 0.25) (layer "F.Cu") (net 53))
 (segment (start 118.364 130.302) (end 118.364 126.492) (width 0.25) (layer "B.Cu") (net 54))
 (segment (start 118.364 126.492) (end 114.554 122.682) (width 0.25) (layer "B.Cu") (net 54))
 (segment (start 114.554 122.682) (end 114.3 122.682) (width 0.25) (layer "B.Cu") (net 54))
 (segment (start 116.469 130.844) (end 117.822 130.844) (width 0.25) (layer "B.Cu") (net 54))
 (segment (start 117.822 130.844) (end 118.364 130.302) (width 0.25) (layer "B.Cu") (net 54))
 (segment (start 114.3 122.682) (end 112.761 121.143) (width 0.25) (layer "B.Cu") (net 54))
 (segment (start 112.761 121.143) (end 109.474 121.143) (width 0.25) (layer "B.Cu") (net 54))
 (segment (start 95.758 136.398) (end 94.234 134.874) (width 1) (layer "B.Cu") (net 11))
 (segment (start 103.124 133.858) (end 103.124 135.636) (width 1) (layer "B.Cu") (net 11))
 (segment (start 118.501 134.991) (end 115.199 134.991) (width 0.25) (layer "B.Cu") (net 11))
 (segment (start 94.234 134.874) (end 94.234 131.303) (width 1) (layer "B.Cu") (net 11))
 (segment (start 118.872 123.19) (end 119.38 123.698) (width 0.25) (layer "B.Cu") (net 11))
 (segment (start 116.332 123.19) (end 118.872 123.19) (width 0.25) (layer "B.Cu") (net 11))
 (segment (start 115.199 122.057) (end 116.332 123.19) (width 0.25) (layer "B.Cu") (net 11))
 (segment (start 113.792 136.398) (end 102.362 136.398) (width 1) (layer "B.Cu") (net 11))
 (segment (start 115.199 132.114) (end 115.199 134.991) (width 1) (layer "B.Cu") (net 11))
 (segment (start 103.124 135.636) (end 102.362 136.398) (width 1) (layer "B.Cu") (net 11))
 (segment (start 119.38 123.698) (end 119.38 134.112) (width 0.25) (layer "B.Cu") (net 11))
 (segment (start 115.199 134.991) (end 113.792 136.398) (width 1) (layer "B.Cu") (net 11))
 (segment (start 102.362 136.398) (end 95.758 136.398) (width 1) (layer "B.Cu") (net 11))
 (segment (start 119.38 134.112) (end 118.501 134.991) (width 0.25) (layer "B.Cu") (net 11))
 (segment (start 115.199 121.221) (end 115.199 122.057) (width 0.25) (layer "B.Cu") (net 11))
 (segment (start 114.808 104.648) (end 115.824 104.648) (width 1) (layer "F.Cu") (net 1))
 (segment (start 114.617 116.141) (end 113.284 114.808) (width 1) (layer "F.Cu") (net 1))
 (segment (start 113.284 106.172) (end 114.808 104.648) (width 1) (layer "F.Cu") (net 1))
 (segment (start 113.284 114.808) (end 113.284 106.172) (width 1) (layer "F.Cu") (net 1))
 (segment (start 115.199 116.141) (end 114.617 116.141) (width 1) (layer "F.Cu") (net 1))
 (segment (start 110.9993 95.743) (end 118.364 103.1077) (width 0.25) (layer "F.Cu") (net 4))
 (segment (start 116.523 116.141) (end 116.469 116.141) (width 0.25) (layer "F.Cu") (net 4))
 (segment (start 118.364 114.3) (end 116.523 116.141) (width 0.25) (layer "F.Cu") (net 4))
 (segment (start 109.474 95.743) (end 110.9993 95.743) (width 0.25) (layer "F.Cu") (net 4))
 (segment (start 118.364 103.1077) (end 118.364 114.3) (width 0.25) (layer "F.Cu") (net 4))
 (segment (start 114.069978 117.411) (end 115.199 117.411) (width 1) (layer "B.Cu") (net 5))
 (segment (start 112.522 115.863022) (end 114.069978 117.411) (width 1) (layer "B.Cu") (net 5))
 (segment (start 112.522 114.554) (end 112.522 115.863022) (width 1) (layer "B.Cu") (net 5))
 (segment (start 109.474 113.523) (end 111.491 113.523) (width 1) (layer "B.Cu") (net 5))
 (segment (start 111.491 113.523) (end 112.522 114.554) (width 1) (layer "B.Cu") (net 5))
 (segment (start 117.602 123.444) (end 118.364 122.682) (width 0.25) (layer "F.Cu") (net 10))
 (segment (start 113.284 123.444) (end 117.602 123.444) (width 0.25) (layer "F.Cu") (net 10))
 (segment (start 118.364 122.682) (end 118.364 120.396) (width 0.25) (layer "F.Cu") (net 10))
 (segment (start 112.522 122.682) (end 113.284 123.444) (width 0.25) (layer "F.Cu") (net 10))
 (segment (start 112.522 119.634) (end 112.522 122.682) (width 0.25) (layer "F.Cu") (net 10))
 (segment (start 111.491 118.603) (end 112.522 119.634) (width 0.25) (layer "F.Cu") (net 10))
 (segment (start 117.919 119.951) (end 118.364 120.396) (width 0.25) (layer "F.Cu") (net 10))
 (segment (start 109.474 118.603) (end 111.491 118.603) (width 0.25) (layer "F.Cu") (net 10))
 (segment (start 116.469 119.951) (end 117.919 119.951) (width 0.25) (layer "F.Cu") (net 10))
 (segment (start 119.38 101.092) (end 115.843 97.555) (width 0.25) (layer "F.Cu") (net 8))
 (segment (start 116.469 118.681) (end 118.809 118.681) (width 0.25) (layer "F.Cu") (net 8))
 (segment (start 115.843 97.555) (end 115.824 97.555) (width 0.25) (layer "F.Cu") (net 8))
 (segment (start 118.809 118.681) (end 119.38 118.11) (width 0.25) (layer "F.Cu") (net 8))
 (segment (start 119.38 118.11) (end 119.38 101.092) (width 0.25) (layer "F.Cu") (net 8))
 (segment (start 96.94947 128.95347) (end 99.314 131.318) (width 0.25) (layer "F.Cu") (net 44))
 (segment (start 95.743 118.603) (end 96.94947 119.80947) (width 0.25) (layer "F.Cu") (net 44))
 (segment (start 94.234 118.603) (end 95.743 118.603) (width 0.25) (layer "F.Cu") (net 44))
 (segment (start 99.314 131.318) (end 100.584 131.318) (width 0.25) (layer "F.Cu") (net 44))
 (segment (start 96.94947 119.80947) (end 96.94947 128.95347) (width 0.25) (layer "F.Cu") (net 44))
 (segment (start 91.44 133.096) (end 91.44 121.92) (width 0.25) (layer "F.Cu") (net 45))
 (segment (start 91.44 121.92) (end 92.217 121.143) (width 0.25) (layer "F.Cu") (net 45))
 (segment (start 100.584 133.858) (end 99.314 135.128) (width 0.25) (layer "F.Cu") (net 45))
 (segment (start 93.472 135.128) (end 91.44 133.096) (width 0.25) (layer "F.Cu") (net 45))
 (segment (start 92.217 121.143) (end 94.234 121.143) (width 0.25) (layer "F.Cu") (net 45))
 (segment (start 99.314 135.128) (end 93.472 135.128) (width 0.25) (layer "F.Cu") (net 45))
 (segment (start 109.474 108.443) (end 113.3937 108.443) (width 1) (layer "B.Cu") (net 2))
 (segment (start 115.824 107.188) (end 114.6487 107.188) (width 1) (layer "B.Cu") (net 2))
 (segment (start 113.3937 108.443) (end 114.6487 107.188) (width 1) (layer "B.Cu") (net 2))
 (segment (start 114.2673 95.015) (end 115.824 95.015) (width 0.25) (layer "B.Cu") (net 55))
 (segment (start 110.9993 98.283) (end 114.2673 95.015) (width 0.25) (layer "B.Cu") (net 55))
 (segment (start 109.474 98.283) (end 110.9993 98.283) (width 0.25) (layer "B.Cu") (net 55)))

